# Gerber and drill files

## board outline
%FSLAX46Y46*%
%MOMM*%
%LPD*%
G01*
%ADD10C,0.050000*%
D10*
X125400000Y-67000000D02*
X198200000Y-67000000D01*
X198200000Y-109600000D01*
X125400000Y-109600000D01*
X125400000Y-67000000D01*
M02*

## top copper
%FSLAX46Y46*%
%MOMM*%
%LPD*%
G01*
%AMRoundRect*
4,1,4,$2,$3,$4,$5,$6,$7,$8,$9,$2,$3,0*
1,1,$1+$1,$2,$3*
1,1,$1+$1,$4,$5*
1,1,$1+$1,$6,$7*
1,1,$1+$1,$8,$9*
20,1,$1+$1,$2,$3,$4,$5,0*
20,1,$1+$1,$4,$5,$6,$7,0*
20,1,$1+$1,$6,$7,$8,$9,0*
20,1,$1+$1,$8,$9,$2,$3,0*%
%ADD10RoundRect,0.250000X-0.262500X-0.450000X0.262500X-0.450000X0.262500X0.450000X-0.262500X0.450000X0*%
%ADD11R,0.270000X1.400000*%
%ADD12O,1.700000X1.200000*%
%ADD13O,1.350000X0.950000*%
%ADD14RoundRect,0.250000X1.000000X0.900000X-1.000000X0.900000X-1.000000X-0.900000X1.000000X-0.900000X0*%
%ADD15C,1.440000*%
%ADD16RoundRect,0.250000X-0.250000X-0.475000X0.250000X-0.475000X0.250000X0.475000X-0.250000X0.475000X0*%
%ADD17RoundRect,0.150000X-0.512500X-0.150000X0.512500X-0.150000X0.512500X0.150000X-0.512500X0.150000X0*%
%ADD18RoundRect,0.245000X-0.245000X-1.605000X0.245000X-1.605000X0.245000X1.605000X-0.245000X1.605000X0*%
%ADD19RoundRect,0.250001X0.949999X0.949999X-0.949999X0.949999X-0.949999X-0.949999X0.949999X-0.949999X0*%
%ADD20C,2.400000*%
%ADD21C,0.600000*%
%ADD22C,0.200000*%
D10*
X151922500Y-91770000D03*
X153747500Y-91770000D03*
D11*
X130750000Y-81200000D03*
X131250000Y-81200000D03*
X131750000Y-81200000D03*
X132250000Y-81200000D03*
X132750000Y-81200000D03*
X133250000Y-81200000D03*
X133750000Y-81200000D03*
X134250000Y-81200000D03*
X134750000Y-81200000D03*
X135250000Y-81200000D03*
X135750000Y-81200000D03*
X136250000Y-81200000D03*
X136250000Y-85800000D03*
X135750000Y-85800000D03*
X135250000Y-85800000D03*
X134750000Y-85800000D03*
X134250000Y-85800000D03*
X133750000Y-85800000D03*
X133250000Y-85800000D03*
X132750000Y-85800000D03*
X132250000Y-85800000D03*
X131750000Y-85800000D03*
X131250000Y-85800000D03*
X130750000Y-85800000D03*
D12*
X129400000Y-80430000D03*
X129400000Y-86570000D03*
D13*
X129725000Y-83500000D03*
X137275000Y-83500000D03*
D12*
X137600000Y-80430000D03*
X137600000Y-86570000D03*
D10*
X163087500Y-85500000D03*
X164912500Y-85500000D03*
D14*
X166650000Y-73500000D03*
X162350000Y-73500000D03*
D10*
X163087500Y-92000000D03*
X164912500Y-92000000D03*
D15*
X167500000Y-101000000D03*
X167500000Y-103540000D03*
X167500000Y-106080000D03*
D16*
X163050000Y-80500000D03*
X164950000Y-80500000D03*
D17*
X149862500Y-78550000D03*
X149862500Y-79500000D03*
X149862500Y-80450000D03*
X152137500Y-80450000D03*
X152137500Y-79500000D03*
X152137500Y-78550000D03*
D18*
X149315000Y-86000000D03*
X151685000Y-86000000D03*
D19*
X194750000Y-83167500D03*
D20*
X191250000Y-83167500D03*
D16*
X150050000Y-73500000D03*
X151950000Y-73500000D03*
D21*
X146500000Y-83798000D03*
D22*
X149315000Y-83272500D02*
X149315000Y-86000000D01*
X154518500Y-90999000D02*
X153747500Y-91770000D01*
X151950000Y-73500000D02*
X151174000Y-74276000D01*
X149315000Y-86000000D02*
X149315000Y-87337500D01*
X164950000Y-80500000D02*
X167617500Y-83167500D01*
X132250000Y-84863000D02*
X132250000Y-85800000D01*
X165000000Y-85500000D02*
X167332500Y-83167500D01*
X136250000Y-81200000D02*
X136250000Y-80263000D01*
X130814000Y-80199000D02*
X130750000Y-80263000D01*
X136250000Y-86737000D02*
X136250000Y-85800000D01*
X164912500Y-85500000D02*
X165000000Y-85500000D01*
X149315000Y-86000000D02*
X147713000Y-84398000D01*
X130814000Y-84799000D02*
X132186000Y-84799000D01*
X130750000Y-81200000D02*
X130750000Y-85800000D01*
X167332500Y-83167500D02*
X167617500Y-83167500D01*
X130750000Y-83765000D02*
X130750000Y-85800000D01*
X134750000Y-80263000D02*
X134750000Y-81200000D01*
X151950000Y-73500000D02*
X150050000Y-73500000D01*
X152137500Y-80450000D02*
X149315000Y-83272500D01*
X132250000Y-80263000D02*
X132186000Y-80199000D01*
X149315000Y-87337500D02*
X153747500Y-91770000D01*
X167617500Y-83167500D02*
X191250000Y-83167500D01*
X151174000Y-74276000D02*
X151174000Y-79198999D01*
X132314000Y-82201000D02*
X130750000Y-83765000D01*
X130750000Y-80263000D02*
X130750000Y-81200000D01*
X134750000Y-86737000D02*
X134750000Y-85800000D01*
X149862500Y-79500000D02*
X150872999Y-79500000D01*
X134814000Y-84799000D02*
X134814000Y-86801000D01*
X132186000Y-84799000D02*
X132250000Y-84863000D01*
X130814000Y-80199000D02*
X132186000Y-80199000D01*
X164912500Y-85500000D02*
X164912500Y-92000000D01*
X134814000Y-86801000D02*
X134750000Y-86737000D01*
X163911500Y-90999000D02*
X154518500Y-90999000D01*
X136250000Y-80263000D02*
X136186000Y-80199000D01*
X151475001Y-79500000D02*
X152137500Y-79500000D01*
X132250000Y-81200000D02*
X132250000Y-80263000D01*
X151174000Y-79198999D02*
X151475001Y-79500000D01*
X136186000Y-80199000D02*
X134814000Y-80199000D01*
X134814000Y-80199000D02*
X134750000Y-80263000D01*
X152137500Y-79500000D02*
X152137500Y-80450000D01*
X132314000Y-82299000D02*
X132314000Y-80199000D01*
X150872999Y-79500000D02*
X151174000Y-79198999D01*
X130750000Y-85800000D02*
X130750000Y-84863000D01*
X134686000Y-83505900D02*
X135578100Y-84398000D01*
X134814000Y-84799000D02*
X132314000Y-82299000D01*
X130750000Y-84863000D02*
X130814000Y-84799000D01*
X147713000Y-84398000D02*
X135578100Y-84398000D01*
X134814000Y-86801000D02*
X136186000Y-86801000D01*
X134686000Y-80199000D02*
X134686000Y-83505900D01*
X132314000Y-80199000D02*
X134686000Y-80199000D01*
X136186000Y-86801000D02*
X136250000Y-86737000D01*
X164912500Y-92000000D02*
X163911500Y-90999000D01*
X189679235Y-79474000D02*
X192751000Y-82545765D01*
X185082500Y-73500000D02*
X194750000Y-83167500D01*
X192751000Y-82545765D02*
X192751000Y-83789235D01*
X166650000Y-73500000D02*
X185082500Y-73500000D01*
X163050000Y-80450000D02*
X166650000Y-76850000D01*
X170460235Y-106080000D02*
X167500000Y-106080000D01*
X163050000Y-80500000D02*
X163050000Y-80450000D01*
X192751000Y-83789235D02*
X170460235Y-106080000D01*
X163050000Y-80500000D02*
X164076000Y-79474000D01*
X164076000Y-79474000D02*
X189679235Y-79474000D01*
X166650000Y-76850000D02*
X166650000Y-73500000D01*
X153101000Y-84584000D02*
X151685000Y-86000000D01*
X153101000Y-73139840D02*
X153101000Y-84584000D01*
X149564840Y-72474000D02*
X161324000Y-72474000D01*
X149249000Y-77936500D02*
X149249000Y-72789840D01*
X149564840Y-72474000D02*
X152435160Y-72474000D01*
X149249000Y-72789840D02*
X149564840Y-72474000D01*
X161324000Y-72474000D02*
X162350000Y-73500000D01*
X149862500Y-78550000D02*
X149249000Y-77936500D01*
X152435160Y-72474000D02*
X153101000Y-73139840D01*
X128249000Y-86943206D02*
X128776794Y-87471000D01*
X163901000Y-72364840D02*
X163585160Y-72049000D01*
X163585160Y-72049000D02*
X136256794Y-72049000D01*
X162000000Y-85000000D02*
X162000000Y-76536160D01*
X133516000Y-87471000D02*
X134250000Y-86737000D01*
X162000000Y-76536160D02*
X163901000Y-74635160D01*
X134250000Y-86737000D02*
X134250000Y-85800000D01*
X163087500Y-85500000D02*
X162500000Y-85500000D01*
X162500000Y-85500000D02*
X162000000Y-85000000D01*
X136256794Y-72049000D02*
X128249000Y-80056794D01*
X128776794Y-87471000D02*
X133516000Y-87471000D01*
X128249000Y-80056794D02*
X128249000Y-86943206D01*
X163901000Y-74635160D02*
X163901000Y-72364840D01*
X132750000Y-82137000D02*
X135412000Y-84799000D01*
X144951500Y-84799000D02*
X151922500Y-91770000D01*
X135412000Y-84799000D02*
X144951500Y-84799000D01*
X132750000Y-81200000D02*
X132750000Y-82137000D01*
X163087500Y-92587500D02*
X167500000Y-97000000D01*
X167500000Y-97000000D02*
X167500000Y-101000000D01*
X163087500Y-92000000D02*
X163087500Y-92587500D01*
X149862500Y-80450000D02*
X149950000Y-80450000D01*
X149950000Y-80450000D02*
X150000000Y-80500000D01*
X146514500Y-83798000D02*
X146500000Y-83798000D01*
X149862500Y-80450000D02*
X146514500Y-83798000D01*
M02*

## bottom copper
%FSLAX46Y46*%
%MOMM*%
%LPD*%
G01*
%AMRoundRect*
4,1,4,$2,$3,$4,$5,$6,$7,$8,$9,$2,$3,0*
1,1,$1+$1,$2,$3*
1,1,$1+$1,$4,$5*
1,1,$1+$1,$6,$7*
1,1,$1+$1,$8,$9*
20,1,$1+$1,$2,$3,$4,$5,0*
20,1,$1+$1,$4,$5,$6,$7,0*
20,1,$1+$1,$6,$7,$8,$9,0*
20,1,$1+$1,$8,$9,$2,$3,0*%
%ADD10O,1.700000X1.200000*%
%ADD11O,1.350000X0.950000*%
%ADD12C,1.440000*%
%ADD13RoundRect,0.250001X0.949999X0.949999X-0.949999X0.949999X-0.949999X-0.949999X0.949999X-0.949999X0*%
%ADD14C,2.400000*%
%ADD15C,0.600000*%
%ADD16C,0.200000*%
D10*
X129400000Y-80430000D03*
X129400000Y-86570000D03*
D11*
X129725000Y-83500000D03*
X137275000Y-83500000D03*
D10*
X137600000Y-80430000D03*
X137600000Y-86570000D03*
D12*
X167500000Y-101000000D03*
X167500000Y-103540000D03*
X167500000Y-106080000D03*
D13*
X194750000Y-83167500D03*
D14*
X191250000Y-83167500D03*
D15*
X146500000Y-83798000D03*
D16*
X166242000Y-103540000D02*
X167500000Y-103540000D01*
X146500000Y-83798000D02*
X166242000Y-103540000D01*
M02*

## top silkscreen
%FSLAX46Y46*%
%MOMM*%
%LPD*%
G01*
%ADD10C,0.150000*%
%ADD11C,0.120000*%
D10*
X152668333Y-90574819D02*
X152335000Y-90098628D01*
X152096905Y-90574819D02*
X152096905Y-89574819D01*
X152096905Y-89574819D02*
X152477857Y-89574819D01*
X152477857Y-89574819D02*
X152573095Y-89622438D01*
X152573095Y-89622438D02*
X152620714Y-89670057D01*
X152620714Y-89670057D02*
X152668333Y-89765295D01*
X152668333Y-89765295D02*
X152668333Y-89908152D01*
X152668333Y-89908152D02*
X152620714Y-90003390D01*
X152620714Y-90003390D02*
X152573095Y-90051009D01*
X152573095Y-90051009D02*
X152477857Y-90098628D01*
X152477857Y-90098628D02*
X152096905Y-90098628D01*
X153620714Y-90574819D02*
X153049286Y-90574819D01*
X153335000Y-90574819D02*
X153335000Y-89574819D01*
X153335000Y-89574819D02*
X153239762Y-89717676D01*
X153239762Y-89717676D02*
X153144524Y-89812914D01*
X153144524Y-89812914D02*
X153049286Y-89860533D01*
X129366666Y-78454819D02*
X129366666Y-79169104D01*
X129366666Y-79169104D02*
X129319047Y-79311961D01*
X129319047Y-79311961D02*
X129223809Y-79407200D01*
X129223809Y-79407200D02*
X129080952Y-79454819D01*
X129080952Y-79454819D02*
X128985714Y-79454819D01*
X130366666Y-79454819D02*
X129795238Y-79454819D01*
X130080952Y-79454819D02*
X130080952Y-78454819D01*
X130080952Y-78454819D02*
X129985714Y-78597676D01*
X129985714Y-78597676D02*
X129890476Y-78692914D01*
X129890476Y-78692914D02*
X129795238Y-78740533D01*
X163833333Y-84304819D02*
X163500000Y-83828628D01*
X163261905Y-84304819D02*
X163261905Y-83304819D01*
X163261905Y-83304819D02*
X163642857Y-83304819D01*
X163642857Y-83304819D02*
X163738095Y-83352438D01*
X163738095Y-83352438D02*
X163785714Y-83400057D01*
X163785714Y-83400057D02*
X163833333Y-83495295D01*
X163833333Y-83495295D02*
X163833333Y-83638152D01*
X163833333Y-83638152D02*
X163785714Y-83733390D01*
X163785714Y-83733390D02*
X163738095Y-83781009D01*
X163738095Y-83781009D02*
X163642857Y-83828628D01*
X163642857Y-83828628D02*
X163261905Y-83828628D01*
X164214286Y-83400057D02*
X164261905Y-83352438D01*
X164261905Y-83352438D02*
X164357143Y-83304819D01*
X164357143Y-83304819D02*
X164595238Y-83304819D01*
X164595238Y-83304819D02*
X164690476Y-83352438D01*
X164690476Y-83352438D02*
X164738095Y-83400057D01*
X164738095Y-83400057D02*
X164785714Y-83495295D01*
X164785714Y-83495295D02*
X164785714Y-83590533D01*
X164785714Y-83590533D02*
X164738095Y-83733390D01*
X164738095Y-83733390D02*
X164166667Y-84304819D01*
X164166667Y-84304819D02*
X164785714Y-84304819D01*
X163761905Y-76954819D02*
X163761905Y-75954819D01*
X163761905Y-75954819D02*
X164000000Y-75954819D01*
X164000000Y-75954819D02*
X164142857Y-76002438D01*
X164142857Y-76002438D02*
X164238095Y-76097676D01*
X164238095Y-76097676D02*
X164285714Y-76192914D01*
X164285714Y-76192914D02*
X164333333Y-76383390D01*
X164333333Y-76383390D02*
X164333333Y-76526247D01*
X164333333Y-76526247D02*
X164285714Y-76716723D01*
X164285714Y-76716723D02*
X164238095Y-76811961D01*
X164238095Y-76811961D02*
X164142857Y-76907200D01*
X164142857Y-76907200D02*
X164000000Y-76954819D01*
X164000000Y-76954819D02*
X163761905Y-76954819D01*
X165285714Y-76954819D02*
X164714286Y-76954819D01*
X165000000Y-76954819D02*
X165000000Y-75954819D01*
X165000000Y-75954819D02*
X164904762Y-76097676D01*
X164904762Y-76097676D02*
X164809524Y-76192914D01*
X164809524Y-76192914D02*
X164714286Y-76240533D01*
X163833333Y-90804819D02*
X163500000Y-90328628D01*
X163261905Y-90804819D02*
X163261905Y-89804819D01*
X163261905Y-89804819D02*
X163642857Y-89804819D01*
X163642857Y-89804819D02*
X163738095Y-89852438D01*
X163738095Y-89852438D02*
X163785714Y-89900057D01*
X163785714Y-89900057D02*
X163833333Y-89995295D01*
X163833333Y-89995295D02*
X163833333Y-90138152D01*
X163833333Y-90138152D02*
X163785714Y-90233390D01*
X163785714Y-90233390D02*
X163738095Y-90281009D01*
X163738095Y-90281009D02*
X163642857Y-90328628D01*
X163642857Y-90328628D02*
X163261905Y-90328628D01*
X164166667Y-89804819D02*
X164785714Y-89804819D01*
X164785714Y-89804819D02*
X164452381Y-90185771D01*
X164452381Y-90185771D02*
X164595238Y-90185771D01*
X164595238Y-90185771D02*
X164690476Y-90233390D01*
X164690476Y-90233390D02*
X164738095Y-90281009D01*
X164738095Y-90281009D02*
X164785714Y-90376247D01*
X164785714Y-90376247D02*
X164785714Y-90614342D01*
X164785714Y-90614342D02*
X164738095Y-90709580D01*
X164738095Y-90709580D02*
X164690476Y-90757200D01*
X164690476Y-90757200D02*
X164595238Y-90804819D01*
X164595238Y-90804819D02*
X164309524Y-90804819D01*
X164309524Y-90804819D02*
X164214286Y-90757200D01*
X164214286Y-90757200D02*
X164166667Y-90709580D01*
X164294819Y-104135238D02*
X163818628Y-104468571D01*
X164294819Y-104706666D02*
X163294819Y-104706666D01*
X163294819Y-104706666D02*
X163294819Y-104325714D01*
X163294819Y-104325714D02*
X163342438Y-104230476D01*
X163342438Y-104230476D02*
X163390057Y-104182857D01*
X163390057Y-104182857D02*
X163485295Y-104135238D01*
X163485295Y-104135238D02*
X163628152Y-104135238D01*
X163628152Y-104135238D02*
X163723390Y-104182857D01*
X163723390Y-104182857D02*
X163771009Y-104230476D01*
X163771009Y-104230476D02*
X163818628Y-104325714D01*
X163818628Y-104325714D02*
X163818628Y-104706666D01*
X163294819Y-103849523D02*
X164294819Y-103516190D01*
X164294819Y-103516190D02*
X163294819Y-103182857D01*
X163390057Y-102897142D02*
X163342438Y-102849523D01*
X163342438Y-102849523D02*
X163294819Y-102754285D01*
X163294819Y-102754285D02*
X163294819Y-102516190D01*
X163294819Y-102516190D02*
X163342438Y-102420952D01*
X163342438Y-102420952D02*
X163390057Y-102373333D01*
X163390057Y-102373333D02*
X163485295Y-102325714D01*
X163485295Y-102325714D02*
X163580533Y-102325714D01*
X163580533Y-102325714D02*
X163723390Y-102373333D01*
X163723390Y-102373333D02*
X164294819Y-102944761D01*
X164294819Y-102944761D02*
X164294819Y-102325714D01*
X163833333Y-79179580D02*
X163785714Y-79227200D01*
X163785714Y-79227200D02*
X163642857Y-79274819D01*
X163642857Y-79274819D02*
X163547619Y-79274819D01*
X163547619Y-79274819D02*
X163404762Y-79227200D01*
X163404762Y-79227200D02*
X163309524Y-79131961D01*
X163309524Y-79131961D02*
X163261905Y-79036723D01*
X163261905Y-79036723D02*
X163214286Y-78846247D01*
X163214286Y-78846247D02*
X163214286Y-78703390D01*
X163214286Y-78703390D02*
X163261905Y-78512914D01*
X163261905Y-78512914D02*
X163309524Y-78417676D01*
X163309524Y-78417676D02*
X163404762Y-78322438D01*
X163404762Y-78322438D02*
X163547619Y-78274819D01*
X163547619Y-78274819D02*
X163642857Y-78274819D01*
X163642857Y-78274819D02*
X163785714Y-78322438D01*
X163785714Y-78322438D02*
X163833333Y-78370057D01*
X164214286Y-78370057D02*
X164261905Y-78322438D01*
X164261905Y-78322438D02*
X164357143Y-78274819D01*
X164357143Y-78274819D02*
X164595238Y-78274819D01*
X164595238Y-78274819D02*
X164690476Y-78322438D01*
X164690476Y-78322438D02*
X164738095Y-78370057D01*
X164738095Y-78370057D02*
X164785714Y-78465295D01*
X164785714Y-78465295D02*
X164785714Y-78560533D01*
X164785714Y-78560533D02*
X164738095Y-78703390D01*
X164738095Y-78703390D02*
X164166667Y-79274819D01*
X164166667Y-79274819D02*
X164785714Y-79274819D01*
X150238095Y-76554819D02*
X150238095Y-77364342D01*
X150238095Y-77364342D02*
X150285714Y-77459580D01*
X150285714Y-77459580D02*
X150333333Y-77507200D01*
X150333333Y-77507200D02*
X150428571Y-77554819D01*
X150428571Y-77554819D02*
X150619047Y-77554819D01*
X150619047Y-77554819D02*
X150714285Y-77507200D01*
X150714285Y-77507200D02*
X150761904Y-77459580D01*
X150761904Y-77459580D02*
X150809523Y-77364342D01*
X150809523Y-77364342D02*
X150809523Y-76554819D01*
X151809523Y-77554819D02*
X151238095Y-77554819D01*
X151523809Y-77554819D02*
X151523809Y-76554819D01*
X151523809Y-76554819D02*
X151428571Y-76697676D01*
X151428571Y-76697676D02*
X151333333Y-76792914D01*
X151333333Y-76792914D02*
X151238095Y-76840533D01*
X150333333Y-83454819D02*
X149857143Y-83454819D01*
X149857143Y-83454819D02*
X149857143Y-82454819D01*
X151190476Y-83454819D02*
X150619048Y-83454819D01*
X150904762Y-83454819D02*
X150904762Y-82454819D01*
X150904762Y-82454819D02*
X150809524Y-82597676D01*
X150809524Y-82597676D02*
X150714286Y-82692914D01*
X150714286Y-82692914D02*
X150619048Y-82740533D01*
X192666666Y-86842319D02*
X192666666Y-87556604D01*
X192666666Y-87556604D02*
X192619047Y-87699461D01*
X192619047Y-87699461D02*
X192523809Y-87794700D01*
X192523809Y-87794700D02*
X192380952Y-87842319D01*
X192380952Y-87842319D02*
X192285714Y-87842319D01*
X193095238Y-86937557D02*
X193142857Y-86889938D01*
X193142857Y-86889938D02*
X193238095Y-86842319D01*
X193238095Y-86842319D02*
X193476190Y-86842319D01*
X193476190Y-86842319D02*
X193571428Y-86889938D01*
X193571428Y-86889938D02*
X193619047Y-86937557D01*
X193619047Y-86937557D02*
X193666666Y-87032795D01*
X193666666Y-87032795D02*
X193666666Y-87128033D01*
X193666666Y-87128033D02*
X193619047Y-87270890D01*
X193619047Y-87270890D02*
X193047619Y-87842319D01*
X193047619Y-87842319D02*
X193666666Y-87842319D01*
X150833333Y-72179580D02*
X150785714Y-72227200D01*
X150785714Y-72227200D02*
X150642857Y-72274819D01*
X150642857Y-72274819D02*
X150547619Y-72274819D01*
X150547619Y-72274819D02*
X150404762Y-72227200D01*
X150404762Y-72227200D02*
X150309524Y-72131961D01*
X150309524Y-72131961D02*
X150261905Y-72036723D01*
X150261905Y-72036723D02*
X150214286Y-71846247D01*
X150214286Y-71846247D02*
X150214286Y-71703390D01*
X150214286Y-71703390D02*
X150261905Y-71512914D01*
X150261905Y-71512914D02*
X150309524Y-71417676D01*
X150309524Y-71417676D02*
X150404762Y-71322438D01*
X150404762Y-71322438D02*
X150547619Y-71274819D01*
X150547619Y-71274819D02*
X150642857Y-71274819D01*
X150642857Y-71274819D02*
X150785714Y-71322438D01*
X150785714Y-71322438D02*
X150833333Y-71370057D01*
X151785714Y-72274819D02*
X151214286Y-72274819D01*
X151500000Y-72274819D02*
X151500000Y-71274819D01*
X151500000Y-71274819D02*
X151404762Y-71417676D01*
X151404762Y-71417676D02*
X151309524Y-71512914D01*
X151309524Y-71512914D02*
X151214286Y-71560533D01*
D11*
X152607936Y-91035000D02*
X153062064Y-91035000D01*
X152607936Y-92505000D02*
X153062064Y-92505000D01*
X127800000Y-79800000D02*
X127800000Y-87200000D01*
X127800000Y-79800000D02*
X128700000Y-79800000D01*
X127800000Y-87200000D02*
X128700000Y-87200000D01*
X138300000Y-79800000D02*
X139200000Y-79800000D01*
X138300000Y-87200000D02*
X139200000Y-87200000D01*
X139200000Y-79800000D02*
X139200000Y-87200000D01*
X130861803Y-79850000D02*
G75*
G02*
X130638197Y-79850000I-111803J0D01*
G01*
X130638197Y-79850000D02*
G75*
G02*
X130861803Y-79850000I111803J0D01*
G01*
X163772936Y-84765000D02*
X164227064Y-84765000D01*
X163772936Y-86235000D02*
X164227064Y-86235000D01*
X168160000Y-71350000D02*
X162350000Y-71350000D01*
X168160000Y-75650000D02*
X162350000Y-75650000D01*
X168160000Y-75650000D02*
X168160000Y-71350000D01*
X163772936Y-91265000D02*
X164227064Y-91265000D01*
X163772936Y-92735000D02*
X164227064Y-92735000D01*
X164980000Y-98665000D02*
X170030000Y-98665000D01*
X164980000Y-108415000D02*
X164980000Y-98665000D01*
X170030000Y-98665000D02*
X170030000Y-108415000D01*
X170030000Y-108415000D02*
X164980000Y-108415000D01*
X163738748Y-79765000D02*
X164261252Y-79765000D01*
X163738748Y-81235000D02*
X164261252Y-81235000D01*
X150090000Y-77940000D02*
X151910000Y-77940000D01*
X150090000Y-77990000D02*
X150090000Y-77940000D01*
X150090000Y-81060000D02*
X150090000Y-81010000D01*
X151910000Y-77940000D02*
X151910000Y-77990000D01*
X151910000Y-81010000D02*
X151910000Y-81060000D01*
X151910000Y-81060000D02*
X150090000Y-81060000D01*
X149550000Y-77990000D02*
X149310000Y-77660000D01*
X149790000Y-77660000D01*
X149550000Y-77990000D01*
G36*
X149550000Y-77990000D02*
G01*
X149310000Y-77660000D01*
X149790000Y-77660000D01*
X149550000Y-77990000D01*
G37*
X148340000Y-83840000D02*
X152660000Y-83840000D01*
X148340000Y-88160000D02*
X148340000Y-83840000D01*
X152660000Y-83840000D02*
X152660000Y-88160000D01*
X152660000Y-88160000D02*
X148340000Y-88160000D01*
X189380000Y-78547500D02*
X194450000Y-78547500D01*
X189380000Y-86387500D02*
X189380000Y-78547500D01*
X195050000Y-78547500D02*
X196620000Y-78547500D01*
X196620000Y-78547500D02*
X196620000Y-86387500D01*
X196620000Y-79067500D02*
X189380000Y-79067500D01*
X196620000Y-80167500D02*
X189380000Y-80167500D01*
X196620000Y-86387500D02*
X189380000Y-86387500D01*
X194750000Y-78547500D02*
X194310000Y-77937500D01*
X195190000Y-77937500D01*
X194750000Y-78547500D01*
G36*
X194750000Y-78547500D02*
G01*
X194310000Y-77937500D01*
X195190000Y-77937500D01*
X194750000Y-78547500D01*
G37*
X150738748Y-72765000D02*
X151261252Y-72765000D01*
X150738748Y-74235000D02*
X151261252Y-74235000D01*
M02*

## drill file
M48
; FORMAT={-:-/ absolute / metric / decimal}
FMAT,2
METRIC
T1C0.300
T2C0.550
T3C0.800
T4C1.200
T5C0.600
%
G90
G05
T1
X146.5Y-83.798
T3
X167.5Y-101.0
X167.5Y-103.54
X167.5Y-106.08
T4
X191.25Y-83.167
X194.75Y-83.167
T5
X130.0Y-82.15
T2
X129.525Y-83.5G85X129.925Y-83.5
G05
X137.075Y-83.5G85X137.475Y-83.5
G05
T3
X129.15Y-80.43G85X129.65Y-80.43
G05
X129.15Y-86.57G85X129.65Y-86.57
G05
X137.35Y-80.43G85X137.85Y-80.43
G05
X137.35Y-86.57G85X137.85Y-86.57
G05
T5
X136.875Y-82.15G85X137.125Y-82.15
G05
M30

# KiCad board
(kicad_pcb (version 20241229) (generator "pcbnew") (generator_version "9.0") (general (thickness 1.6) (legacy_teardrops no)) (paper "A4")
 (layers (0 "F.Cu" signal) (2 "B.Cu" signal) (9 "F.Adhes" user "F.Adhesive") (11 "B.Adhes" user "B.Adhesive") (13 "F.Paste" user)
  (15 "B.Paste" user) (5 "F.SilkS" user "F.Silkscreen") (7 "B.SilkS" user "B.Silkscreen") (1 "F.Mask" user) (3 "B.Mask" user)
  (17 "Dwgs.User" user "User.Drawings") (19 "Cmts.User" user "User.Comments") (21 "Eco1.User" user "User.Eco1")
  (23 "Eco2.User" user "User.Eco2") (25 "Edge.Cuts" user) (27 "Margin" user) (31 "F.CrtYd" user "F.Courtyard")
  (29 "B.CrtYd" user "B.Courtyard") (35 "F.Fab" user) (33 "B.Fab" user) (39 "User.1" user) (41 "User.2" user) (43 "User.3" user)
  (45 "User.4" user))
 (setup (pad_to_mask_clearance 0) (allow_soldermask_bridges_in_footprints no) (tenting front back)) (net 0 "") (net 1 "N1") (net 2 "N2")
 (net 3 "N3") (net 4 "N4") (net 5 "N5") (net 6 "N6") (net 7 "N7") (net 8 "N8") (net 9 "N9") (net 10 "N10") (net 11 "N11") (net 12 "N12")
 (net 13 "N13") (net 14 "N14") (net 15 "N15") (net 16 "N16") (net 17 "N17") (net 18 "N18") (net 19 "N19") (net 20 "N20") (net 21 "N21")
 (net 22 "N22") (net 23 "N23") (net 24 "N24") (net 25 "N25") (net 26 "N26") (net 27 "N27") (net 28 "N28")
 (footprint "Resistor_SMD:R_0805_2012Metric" (layer "F.Cu") (at 152.835 91.77)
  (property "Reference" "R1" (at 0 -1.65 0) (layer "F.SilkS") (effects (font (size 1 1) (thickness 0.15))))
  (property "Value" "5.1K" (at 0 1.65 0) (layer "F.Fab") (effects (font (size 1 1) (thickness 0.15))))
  (fp_line (start -0.227064 -0.735) (end 0.227064 -0.735) (stroke (width 0.12) (type solid)) (layer "F.SilkS"))
  (fp_line (start -0.227064 0.735) (end 0.227064 0.735) (stroke (width 0.12) (type solid)) (layer "F.SilkS"))
  (pad "1" smd roundrect (at -0.9125 0) (size 1.025 1.4) (layers "F.Cu" "F.Mask" "F.Paste") (roundrect_rratio 0.243902) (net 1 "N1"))
  (pad "2" smd roundrect (at 0.9125 0) (size 1.025 1.4) (layers "F.Cu" "F.Mask" "F.Paste") (roundrect_rratio 0.243902) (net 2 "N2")))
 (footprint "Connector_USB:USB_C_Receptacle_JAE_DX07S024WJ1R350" (layer "F.Cu") (at 133.5 83.5)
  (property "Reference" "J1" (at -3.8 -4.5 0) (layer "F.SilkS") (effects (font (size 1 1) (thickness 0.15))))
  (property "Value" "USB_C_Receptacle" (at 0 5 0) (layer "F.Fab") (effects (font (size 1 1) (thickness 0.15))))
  (fp_line (start -5.7 -3.7) (end -5.7 3.7) (stroke (width 0.12) (type solid)) (layer "F.SilkS"))
  (fp_line (start -5.7 -3.7) (end -4.8 -3.7) (stroke (width 0.12) (type solid)) (layer "F.SilkS"))
  (fp_line (start -5.7 3.7) (end -4.8 3.7) (stroke (width 0.12) (type solid)) (layer "F.SilkS"))
  (fp_line (start 4.8 -3.7) (end 5.7 -3.7) (stroke (width 0.12) (type solid)) (layer "F.SilkS"))
  (fp_line (start 4.8 3.7) (end 5.7 3.7) (stroke (width 0.12) (type solid)) (layer "F.SilkS"))
  (fp_line (start 5.7 -3.7) (end 5.7 3.7) (stroke (width 0.12) (type solid)) (layer "F.SilkS"))
  (fp_circle (center -2.75 -3.65) (end -2.638197 -3.65) (stroke (width 0.12) (type solid)) (fill no) (layer "F.SilkS"))
  (pad "" np_thru_hole circle (at -3.5 -1.35) (size 0.6 0.6) (drill 0.6) (layers "*.Cu" "*.Mask"))
  (pad "" np_thru_hole oval (at 3.5 -1.35) (size 0.85 0.6) (drill oval 0.85 0.6) (layers "*.Cu" "*.Mask"))
  (pad "A1" smd rect (at -2.75 -2.3) (size 0.27 1.4) (layers "F.Cu" "F.Mask" "F.Paste") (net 2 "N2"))
  (pad "A2" smd rect (at -2.25 -2.3) (size 0.27 1.4) (layers "F.Cu" "F.Mask" "F.Paste") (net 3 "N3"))
  (pad "A3" smd rect (at -1.75 -2.3) (size 0.27 1.4) (layers "F.Cu" "F.Mask" "F.Paste") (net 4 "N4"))
  (pad "A4" smd rect (at -1.25 -2.3) (size 0.27 1.4) (layers "F.Cu" "F.Mask" "F.Paste") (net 2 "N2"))
  (pad "A5" smd rect (at -0.75 -2.3) (size 0.27 1.4) (layers "F.Cu" "F.Mask" "F.Paste") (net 1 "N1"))
  (pad "A6" smd rect (at -0.25 -2.3) (size 0.27 1.4) (layers "F.Cu" "F.Mask" "F.Paste") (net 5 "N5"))
  (pad "A7" smd rect (at 0.25 -2.3) (size 0.27 1.4) (layers "F.Cu" "F.Mask" "F.Paste") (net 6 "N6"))
  (pad "A8" smd rect (at 0.75 -2.3) (size 0.27 1.4) (layers "F.Cu" "F.Mask" "F.Paste") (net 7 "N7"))
  (pad "A9" smd rect (at 1.25 -2.3) (size 0.27 1.4) (layers "F.Cu" "F.Mask" "F.Paste") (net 2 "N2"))
  (pad "A10" smd rect (at 1.75 -2.3) (size 0.27 1.4) (layers "F.Cu" "F.Mask" "F.Paste") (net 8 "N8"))
  (pad "A11" smd rect (at 2.25 -2.3) (size 0.27 1.4) (layers "F.Cu" "F.Mask" "F.Paste") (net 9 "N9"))
  (pad "A12" smd rect (at 2.75 -2.3) (size 0.27 1.4) (layers "F.Cu" "F.Mask" "F.Paste") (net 2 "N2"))
  (pad "B1" smd rect (at 2.75 2.3) (size 0.27 1.4) (layers "F.Cu" "F.Mask" "F.Paste") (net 2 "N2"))
  (pad "B2" smd rect (at 2.25 2.3) (size 0.27 1.4) (layers "F.Cu" "F.Mask" "F.Paste") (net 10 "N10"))
  (pad "B3" smd rect (at 1.75 2.3) (size 0.27 1.4) (layers "F.Cu" "F.Mask" "F.Paste") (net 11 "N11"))
  (pad "B4" smd rect (at 1.25 2.3) (size 0.27 1.4) (layers "F.Cu" "F.Mask" "F.Paste") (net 2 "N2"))
  (pad "B5" smd rect (at 0.75 2.3) (size 0.27 1.4) (layers "F.Cu" "F.Mask" "F.Paste") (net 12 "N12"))
  (pad "B6" smd rect (at 0.25 2.3) (size 0.27 1.4) (layers "F.Cu" "F.Mask" "F.Paste") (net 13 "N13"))
  (pad "B7" smd rect (at -0.25 2.3) (size 0.27 1.4) (layers "F.Cu" "F.Mask" "F.Paste") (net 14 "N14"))
  (pad "B8" smd rect (at -0.75 2.3) (size 0.27 1.4) (layers "F.Cu" "F.Mask" "F.Paste") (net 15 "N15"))
  (pad "B9" smd rect (at -1.25 2.3) (size 0.27 1.4) (layers "F.Cu" "F.Mask" "F.Paste") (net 2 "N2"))
  (pad "B10" smd rect (at -1.75 2.3) (size 0.27 1.4) (layers "F.Cu" "F.Mask" "F.Paste") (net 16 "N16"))
  (pad "B11" smd rect (at -2.25 2.3) (size 0.27 1.4) (layers "F.Cu" "F.Mask" "F.Paste") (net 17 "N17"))
  (pad "B12" smd rect (at -2.75 2.3) (size 0.27 1.4) (layers "F.Cu" "F.Mask" "F.Paste") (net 2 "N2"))
  (pad "S1" thru_hole oval (at -4.1 -3.07 90) (size 1.2 1.7) (drill oval 0.8 1.3) (layers "*.Cu" "*.Mask") (remove_unused_layers no)
   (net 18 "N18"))
  (pad "S1" thru_hole oval (at -4.1 3.07 90) (size 1.2 1.7) (drill oval 0.8 1.3) (layers "*.Cu" "*.Mask") (remove_unused_layers no)
   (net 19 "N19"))
  (pad "S1" thru_hole oval (at -3.775 0 90) (size 0.95 1.35) (drill oval 0.55 0.95) (layers "*.Cu" "*.Mask") (remove_unused_layers no)
   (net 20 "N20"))
  (pad "S1" thru_hole oval (at 3.775 0 90) (size 0.95 1.35) (drill oval 0.55 0.95) (layers "*.Cu" "*.Mask") (remove_unused_layers no)
   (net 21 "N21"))
  (pad "S1" thru_hole oval (at 4.1 -3.07 90) (size 1.2 1.7) (drill oval 0.8 1.3) (layers "*.Cu" "*.Mask") (remove_unused_layers no)
   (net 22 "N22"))
  (pad "S1" thru_hole oval (at 4.1 3.07 90) (size 1.2 1.7) (drill oval 0.8 1.3) (layers "*.Cu" "*.Mask") (remove_unused_layers no)
   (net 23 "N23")))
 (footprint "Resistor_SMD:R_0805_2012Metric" (layer "F.Cu") (at 164 85.5)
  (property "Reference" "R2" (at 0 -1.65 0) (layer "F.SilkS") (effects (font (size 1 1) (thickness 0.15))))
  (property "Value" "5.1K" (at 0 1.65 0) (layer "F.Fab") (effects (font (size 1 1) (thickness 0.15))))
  (fp_line (start -0.227064 -0.735) (end 0.227064 -0.735) (stroke (width 0.12) (type solid)) (layer "F.SilkS"))
  (fp_line (start -0.227064 0.735) (end 0.227064 0.735) (stroke (width 0.12) (type solid)) (layer "F.SilkS"))
  (pad "1" smd roundrect (at -0.9125 0) (size 1.025 1.4) (layers "F.Cu" "F.Mask" "F.Paste") (roundrect_rratio 0.243902) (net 12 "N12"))
  (pad "2" smd roundrect (at 0.9125 0) (size 1.025 1.4) (layers "F.Cu" "F.Mask" "F.Paste") (roundrect_rratio 0.243902) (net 2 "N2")))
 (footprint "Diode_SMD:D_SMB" (layer "F.Cu") (at 164.5 73.5 180)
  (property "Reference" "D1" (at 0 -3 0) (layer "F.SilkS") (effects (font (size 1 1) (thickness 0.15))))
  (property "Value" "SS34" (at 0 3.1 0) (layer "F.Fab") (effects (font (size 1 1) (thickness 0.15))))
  (fp_line (start -3.66 2.15) (end 2.15 2.15) (stroke (width 0.12) (type solid)) (layer "F.SilkS"))
  (fp_line (start -3.66 -2.15) (end 2.15 -2.15) (stroke (width 0.12) (type solid)) (layer "F.SilkS"))
  (fp_line (start -3.66 -2.15) (end -3.66 2.15) (stroke (width 0.12) (type solid)) (layer "F.SilkS"))
  (pad "1" smd roundrect (at -2.15 0 180) (size 2.5 2.3) (layers "F.Cu" "F.Mask" "F.Paste") (roundrect_rratio 0.1086956522) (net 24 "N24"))
  (pad "2" smd roundrect (at 2.15 0 180) (size 2.5 2.3) (layers "F.Cu" "F.Mask" "F.Paste") (roundrect_rratio 0.1086956522) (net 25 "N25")))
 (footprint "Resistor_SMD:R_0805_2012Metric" (layer "F.Cu") (at 164 92)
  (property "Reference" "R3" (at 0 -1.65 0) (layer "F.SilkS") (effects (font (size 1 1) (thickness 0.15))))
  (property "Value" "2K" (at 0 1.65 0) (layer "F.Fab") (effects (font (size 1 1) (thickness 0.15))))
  (fp_line (start -0.227064 -0.735) (end 0.227064 -0.735) (stroke (width 0.12) (type solid)) (layer "F.SilkS"))
  (fp_line (start -0.227064 0.735) (end 0.227064 0.735) (stroke (width 0.12) (type solid)) (layer "F.SilkS"))
  (pad "1" smd roundrect (at -0.9125 0) (size 1.025 1.4) (layers "F.Cu" "F.Mask" "F.Paste") (roundrect_rratio 0.243902) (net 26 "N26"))
  (pad "2" smd roundrect (at 0.9125 0) (size 1.025 1.4) (layers "F.Cu" "F.Mask" "F.Paste") (roundrect_rratio 0.243902) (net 2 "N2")))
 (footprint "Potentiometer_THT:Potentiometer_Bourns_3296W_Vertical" (layer "F.Cu") (at 167.5 101 90)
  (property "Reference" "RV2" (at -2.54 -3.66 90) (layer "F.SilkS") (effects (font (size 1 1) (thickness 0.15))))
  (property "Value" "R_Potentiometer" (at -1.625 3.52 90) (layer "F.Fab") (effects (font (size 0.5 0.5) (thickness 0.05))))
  (fp_line (start 2.335 -2.52) (end 2.335 2.53) (stroke (width 0.12) (type solid)) (layer "F.SilkS"))
  (fp_line (start -7.415 -2.52) (end 2.335 -2.52) (stroke (width 0.12) (type solid)) (layer "F.SilkS"))
  (fp_line (start 2.335 2.53) (end -7.415 2.53) (stroke (width 0.12) (type solid)) (layer "F.SilkS"))
  (fp_line (start -7.415 2.53) (end -7.415 -2.52) (stroke (width 0.12) (type solid)) (layer "F.SilkS"))
  (pad "1" thru_hole circle (at 0 0 90) (size 1.44 1.44) (drill 0.8) (layers "*.Cu" "*.Mask") (remove_unused_layers no) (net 26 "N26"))
  (pad "2" thru_hole circle (at -2.54 0 90) (size 1.44 1.44) (drill 0.8) (layers "*.Cu" "*.Mask") (remove_unused_layers no) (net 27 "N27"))
  (pad "3" thru_hole circle (at -5.08 0 90) (size 1.44 1.44) (drill 0.8) (layers "*.Cu" "*.Mask") (remove_unused_layers no) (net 24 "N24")))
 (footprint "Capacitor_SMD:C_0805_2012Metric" (layer "F.Cu") (at 164 80.5)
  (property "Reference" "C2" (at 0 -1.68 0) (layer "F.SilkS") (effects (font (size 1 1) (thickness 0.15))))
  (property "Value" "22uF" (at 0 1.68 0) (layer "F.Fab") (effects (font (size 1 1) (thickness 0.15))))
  (fp_line (start -0.261252 -0.735) (end 0.261252 -0.735) (stroke (width 0.12) (type solid)) (layer "F.SilkS"))
  (fp_line (start -0.261252 0.735) (end 0.261252 0.735) (stroke (width 0.12) (type solid)) (layer "F.SilkS"))
  (pad "1" smd roundrect (at -0.95 0) (size 1 1.45) (layers "F.Cu" "F.Mask" "F.Paste") (roundrect_rratio 0.25) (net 24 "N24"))
  (pad "2" smd roundrect (at 0.95 0) (size 1 1.45) (layers "F.Cu" "F.Mask" "F.Paste") (roundrect_rratio 0.25) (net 2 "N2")))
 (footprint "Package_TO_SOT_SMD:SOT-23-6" (layer "F.Cu") (at 151 79.5)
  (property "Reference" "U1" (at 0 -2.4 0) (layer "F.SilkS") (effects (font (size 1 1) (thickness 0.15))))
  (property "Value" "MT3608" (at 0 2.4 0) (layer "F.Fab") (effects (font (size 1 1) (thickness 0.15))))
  (fp_line (start -0.91 -1.56) (end 0.91 -1.56) (stroke (width 0.12) (type solid)) (layer "F.SilkS"))
  (fp_line (start -0.91 -1.51) (end -0.91 -1.56) (stroke (width 0.12) (type solid)) (layer "F.SilkS"))
  (fp_line (start -0.91 1.56) (end -0.91 1.51) (stroke (width 0.12) (type solid)) (layer "F.SilkS"))
  (fp_line (start 0.91 -1.56) (end 0.91 -1.51) (stroke (width 0.12) (type solid)) (layer "F.SilkS"))
  (fp_line (start 0.91 1.51) (end 0.91 1.56) (stroke (width 0.12) (type solid)) (layer "F.SilkS"))
  (fp_line (start 0.91 1.56) (end -0.91 1.56) (stroke (width 0.12) (type solid)) (layer "F.SilkS"))
  (fp_poly (pts (xy -1.45 -1.51) (xy -1.69 -1.84) (xy -1.21 -1.84)) (stroke (width 0.12) (type solid)) (fill yes) (layer "F.SilkS"))
  (pad "1" smd roundrect (at -1.1375 -0.95) (size 1.325 0.6) (layers "F.Cu" "F.Mask" "F.Paste") (roundrect_rratio 0.25) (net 25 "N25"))
  (pad "2" smd roundrect (at -1.1375 0) (size 1.325 0.6) (layers "F.Cu" "F.Mask" "F.Paste") (roundrect_rratio 0.25) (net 2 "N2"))
  (pad "3" smd roundrect (at -1.1375 0.95) (size 1.325 0.6) (layers "F.Cu" "F.Mask" "F.Paste") (roundrect_rratio 0.25) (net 27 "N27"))
  (pad "4" smd roundrect (at 1.1375 0.95) (size 1.325 0.6) (layers "F.Cu" "F.Mask" "F.Paste") (roundrect_rratio 0.25) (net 2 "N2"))
  (pad "5" smd roundrect (at 1.1375 0) (size 1.325 0.6) (layers "F.Cu" "F.Mask" "F.Paste") (roundrect_rratio 0.25) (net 2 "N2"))
  (pad "6" smd roundrect (at 1.1375 -0.95) (size 1.325 0.6) (layers "F.Cu" "F.Mask" "F.Paste") (roundrect_rratio 0.25) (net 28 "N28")))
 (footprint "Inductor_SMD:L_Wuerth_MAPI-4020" (layer "F.Cu") (at 150.5 86)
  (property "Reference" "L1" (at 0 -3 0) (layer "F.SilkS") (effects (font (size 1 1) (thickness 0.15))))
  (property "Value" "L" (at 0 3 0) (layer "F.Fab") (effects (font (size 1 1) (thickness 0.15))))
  (fp_line (start -2.16 -2.16) (end 2.16 -2.16) (stroke (width 0.12) (type solid)) (layer "F.SilkS"))
  (fp_line (start -2.16 2.16) (end -2.16 -2.16) (stroke (width 0.12) (type solid)) (layer "F.SilkS"))
  (fp_line (start 2.16 -2.16) (end 2.16 2.16) (stroke (width 0.12) (type solid)) (layer "F.SilkS"))
  (fp_line (start 2.16 2.16) (end -2.16 2.16) (stroke (width 0.12) (type solid)) (layer "F.SilkS"))
  (pad "1" smd roundrect (at -1.185 0) (size 0.98 3.7) (layers "F.Cu" "F.Mask" "F.Paste") (roundrect_rratio 0.25) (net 2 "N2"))
  (pad "2" smd roundrect (at 1.185 0) (size 0.98 3.7) (layers "F.Cu" "F.Mask" "F.Paste") (roundrect_rratio 0.25) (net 25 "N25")))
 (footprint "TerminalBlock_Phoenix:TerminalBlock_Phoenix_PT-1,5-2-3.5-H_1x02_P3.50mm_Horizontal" (layer "F.Cu") (at 194.75 83.1675 180)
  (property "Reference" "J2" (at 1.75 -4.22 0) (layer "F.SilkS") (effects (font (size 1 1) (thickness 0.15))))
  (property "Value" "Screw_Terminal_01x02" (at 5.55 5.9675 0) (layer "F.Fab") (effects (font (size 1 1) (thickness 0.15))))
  (fp_line (start 5.37 4.62) (end 0.3 4.62) (stroke (width 0.12) (type solid)) (layer "F.SilkS"))
  (fp_line (start 5.37 -3.22) (end 5.37 4.62) (stroke (width 0.12) (type solid)) (layer "F.SilkS"))
  (fp_line (start -0.3 4.62) (end -1.87 4.62) (stroke (width 0.12) (type solid)) (layer "F.SilkS"))
  (fp_line (start -1.87 4.62) (end -1.87 -3.22) (stroke (width 0.12) (type solid)) (layer "F.SilkS"))
  (fp_line (start -1.87 4.1) (end 5.37 4.1) (stroke (width 0.12) (type solid)) (layer "F.SilkS"))
  (fp_line (start -1.87 3) (end 5.37 3) (stroke (width 0.12) (type solid)) (layer "F.SilkS"))
  (fp_line (start -1.87 -3.22) (end 5.37 -3.22) (stroke (width 0.12) (type solid)) (layer "F.SilkS"))
  (fp_poly (pts (xy 0 4.62) (xy 0.44 5.23) (xy -0.44 5.23)) (stroke (width 0.12) (type solid)) (fill yes) (layer "F.SilkS"))
  (pad "1" thru_hole roundrect (at 0 0 180) (size 2.4 2.4) (drill 1.2) (layers "*.Cu" "*.Mask") (remove_unused_layers no)
   (roundrect_rratio 0.104167) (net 24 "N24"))
  (pad "2" thru_hole circle (at 3.5 0 180) (size 2.4 2.4) (drill 1.2) (layers "*.Cu" "*.Mask") (remove_unused_layers no) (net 2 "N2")))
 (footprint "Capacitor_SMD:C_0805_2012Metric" (layer "F.Cu") (at 151 73.5)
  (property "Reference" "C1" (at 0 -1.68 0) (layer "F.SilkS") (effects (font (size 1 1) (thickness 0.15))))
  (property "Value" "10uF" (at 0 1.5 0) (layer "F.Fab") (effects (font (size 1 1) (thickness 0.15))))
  (fp_line (start -0.261252 -0.735) (end 0.261252 -0.735) (stroke (width 0.12) (type solid)) (layer "F.SilkS"))
  (fp_line (start -0.261252 0.735) (end 0.261252 0.735) (stroke (width 0.12) (type solid)) (layer "F.SilkS"))
  (pad "1" smd roundrect (at -0.95 0) (size 1 1.45) (layers "F.Cu" "F.Mask" "F.Paste") (roundrect_rratio 0.25) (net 2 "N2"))
  (pad "2" smd roundrect (at 0.95 0) (size 1 1.45) (layers "F.Cu" "F.Mask" "F.Paste") (roundrect_rratio 0.25) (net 2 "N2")))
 (gr_rect (start 125.4 67) (end 198.2 109.6) (stroke (width 0.05) (type default)) (fill no) (layer "Edge.Cuts"))
 (segment (start 149.315 83.2725) (end 149.315 86) (width 0.2) (layer "F.Cu") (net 2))
 (segment (start 154.5185 90.999) (end 153.7475 91.77) (width 0.2) (layer "F.Cu") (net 2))
 (segment (start 151.95 73.5) (end 151.174 74.276) (width 0.2) (layer "F.Cu") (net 2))
 (segment (start 149.315 86) (end 149.315 87.3375) (width 0.2) (layer "F.Cu") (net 2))
 (segment (start 164.95 80.5) (end 167.6175 83.1675) (width 0.2) (layer "F.Cu") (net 2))
 (segment (start 132.25 84.863) (end 132.25 85.8) (width 0.2) (layer "F.Cu") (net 2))
 (segment (start 165 85.5) (end 167.3325 83.1675) (width 0.2) (layer "F.Cu") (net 2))
 (segment (start 136.25 81.2) (end 136.25 80.263) (width 0.2) (layer "F.Cu") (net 2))
 (segment (start 130.814 80.199) (end 130.75 80.263) (width 0.2) (layer "F.Cu") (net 2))
 (segment (start 136.25 86.737) (end 136.25 85.8) (width 0.2) (layer "F.Cu") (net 2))
 (segment (start 164.9125 85.5) (end 165 85.5) (width 0.2) (layer "F.Cu") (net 2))
 (segment (start 149.315 86) (end 147.713 84.398) (width 0.2) (layer "F.Cu") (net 2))
 (segment (start 130.814 84.799) (end 132.186 84.799) (width 0.2) (layer "F.Cu") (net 2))
 (segment (start 130.75 81.2) (end 130.75 85.8) (width 0.2) (layer "F.Cu") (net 2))
 (segment (start 167.3325 83.1675) (end 167.6175 83.1675) (width 0.2) (layer "F.Cu") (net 2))
 (segment (start 130.75 83.765) (end 130.75 85.8) (width 0.2) (layer "F.Cu") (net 2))
 (segment (start 134.75 80.263) (end 134.75 81.2) (width 0.2) (layer "F.Cu") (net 2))
 (segment (start 151.95 73.5) (end 150.05 73.5) (width 0.2) (layer "F.Cu") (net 2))
 (segment (start 152.1375 80.45) (end 149.315 83.2725) (width 0.2) (layer "F.Cu") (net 2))
 (segment (start 132.25 80.263) (end 132.186 80.199) (width 0.2) (layer "F.Cu") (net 2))
 (segment (start 149.315 87.3375) (end 153.7475 91.77) (width 0.2) (layer "F.Cu") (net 2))
 (segment (start 167.6175 83.1675) (end 191.25 83.1675) (width 0.2) (layer "F.Cu") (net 2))
 (segment (start 151.174 74.276) (end 151.174 79.198999) (width 0.2) (layer "F.Cu") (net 2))
 (segment (start 132.314 82.201) (end 130.75 83.765) (width 0.2) (layer "F.Cu") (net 2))
 (segment (start 130.75 80.263) (end 130.75 81.2) (width 0.2) (layer "F.Cu") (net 2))
 (segment (start 134.75 86.737) (end 134.75 85.8) (width 0.2) (layer "F.Cu") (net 2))
 (segment (start 149.8625 79.5) (end 150.872999 79.5) (width 0.2) (layer "F.Cu") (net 2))
 (segment (start 134.814 84.799) (end 134.814 86.801) (width 0.2) (layer "F.Cu") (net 2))
 (segment (start 132.186 84.799) (end 132.25 84.863) (width 0.2) (layer "F.Cu") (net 2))
 (segment (start 130.814 80.199) (end 132.186 80.199) (width 0.2) (layer "F.Cu") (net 2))
 (segment (start 164.9125 85.5) (end 164.9125 92) (width 0.2) (layer "F.Cu") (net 2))
 (segment (start 134.814 86.801) (end 134.75 86.737) (width 0.2) (layer "F.Cu") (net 2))
 (segment (start 163.9115 90.999) (end 154.5185 90.999) (width 0.2) (layer "F.Cu") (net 2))
 (segment (start 136.25 80.263) (end 136.186 80.199) (width 0.2) (layer "F.Cu") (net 2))
 (segment (start 151.475001 79.5) (end 152.1375 79.5) (width 0.2) (layer "F.Cu") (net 2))
 (segment (start 132.25 81.2) (end 132.25 80.263) (width 0.2) (layer "F.Cu") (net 2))
 (segment (start 151.174 79.198999) (end 151.475001 79.5) (width 0.2) (layer "F.Cu") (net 2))
 (segment (start 136.186 80.199) (end 134.814 80.199) (width 0.2) (layer "F.Cu") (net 2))
 (segment (start 134.814 80.199) (end 134.75 80.263) (width 0.2) (layer "F.Cu") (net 2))
 (segment (start 152.1375 79.5) (end 152.1375 80.45) (width 0.2) (layer "F.Cu") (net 2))
 (segment (start 132.314 82.299) (end 132.314 80.199) (width 0.2) (layer "F.Cu") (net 2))
 (segment (start 150.872999 79.5) (end 151.174 79.198999) (width 0.2) (layer "F.Cu") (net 2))
 (segment (start 130.75 85.8) (end 130.75 84.863) (width 0.2) (layer "F.Cu") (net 2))
 (segment (start 134.686 83.5059) (end 135.5781 84.398) (width 0.2) (layer "F.Cu") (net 2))
 (segment (start 134.814 84.799) (end 132.314 82.299) (width 0.2) (layer "F.Cu") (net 2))
 (segment (start 130.75 84.863) (end 130.814 84.799) (width 0.2) (layer "F.Cu") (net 2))
 (segment (start 147.713 84.398) (end 135.5781 84.398) (width 0.2) (layer "F.Cu") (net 2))
 (segment (start 134.814 86.801) (end 136.186 86.801) (width 0.2) (layer "F.Cu") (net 2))
 (segment (start 134.686 80.199) (end 134.686 83.5059) (width 0.2) (layer "F.Cu") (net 2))
 (segment (start 132.314 80.199) (end 134.686 80.199) (width 0.2) (layer "F.Cu") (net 2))
 (segment (start 136.186 86.801) (end 136.25 86.737) (width 0.2) (layer "F.Cu") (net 2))
 (segment (start 164.9125 92) (end 163.9115 90.999) (width 0.2) (layer "F.Cu") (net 2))
 (segment (start 189.679235 79.474) (end 192.751 82.545765) (width 0.2) (layer "F.Cu") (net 24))
 (segment (start 185.0825 73.5) (end 194.75 83.1675) (width 0.2) (layer "F.Cu") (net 24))
 (segment (start 192.751 82.545765) (end 192.751 83.789235) (width 0.2) (layer "F.Cu") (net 24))
 (segment (start 166.65 73.5) (end 185.0825 73.5) (width 0.2) (layer "F.Cu") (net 24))
 (segment (start 163.05 80.45) (end 166.65 76.85) (width 0.2) (layer "F.Cu") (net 24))
 (segment (start 170.460235 106.08) (end 167.5 106.08) (width 0.2) (layer "F.Cu") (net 24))
 (segment (start 163.05 80.5) (end 163.05 80.45) (width 0.2) (layer "F.Cu") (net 24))
 (segment (start 192.751 83.789235) (end 170.460235 106.08) (width 0.2) (layer "F.Cu") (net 24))
 (segment (start 163.05 80.5) (end 164.076 79.474) (width 0.2) (layer "F.Cu") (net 24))
 (segment (start 164.076 79.474) (end 189.679235 79.474) (width 0.2) (layer "F.Cu") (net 24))
 (segment (start 166.65 76.85) (end 166.65 73.5) (width 0.2) (layer "F.Cu") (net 24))
 (segment (start 153.101 84.584) (end 151.685 86) (width 0.2) (layer "F.Cu") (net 25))
 (segment (start 153.101 73.13984) (end 153.101 84.584) (width 0.2) (layer "F.Cu") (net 25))
 (segment (start 149.56484 72.474) (end 161.324 72.474) (width 0.2) (layer "F.Cu") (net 25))
 (segment (start 149.249 77.9365) (end 149.249 72.78984) (width 0.2) (layer "F.Cu") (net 25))
 (segment (start 149.56484 72.474) (end 152.43516 72.474) (width 0.2) (layer "F.Cu") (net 25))
 (segment (start 149.249 72.78984) (end 149.56484 72.474) (width 0.2) (layer "F.Cu") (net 25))
 (segment (start 161.324 72.474) (end 162.35 73.5) (width 0.2) (layer "F.Cu") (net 25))
 (segment (start 149.8625 78.55) (end 149.249 77.9365) (width 0.2) (layer "F.Cu") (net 25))
 (segment (start 152.43516 72.474) (end 153.101 73.13984) (width 0.2) (layer "F.Cu") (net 25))
 (segment (start 128.249 86.943206) (end 128.776794 87.471) (width 0.2) (layer "F.Cu") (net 12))
 (segment (start 163.901 72.36484) (end 163.58516 72.049) (width 0.2) (layer "F.Cu") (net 12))
 (segment (start 163.58516 72.049) (end 136.256794 72.049) (width 0.2) (layer "F.Cu") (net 12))
 (segment (start 162 85) (end 162 76.53616) (width 0.2) (layer "F.Cu") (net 12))
 (segment (start 133.516 87.471) (end 134.25 86.737) (width 0.2) (layer "F.Cu") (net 12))
 (segment (start 162 76.53616) (end 163.901 74.63516) (width 0.2) (layer "F.Cu") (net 12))
 (segment (start 134.25 86.737) (end 134.25 85.8) (width 0.2) (layer "F.Cu") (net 12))
 (segment (start 163.0875 85.5) (end 162.5 85.5) (width 0.2) (layer "F.Cu") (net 12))
 (segment (start 162.5 85.5) (end 162 85) (width 0.2) (layer "F.Cu") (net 12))
 (segment (start 136.256794 72.049) (end 128.249 80.056794) (width 0.2) (layer "F.Cu") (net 12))
 (segment (start 128.776794 87.471) (end 133.516 87.471) (width 0.2) (layer "F.Cu") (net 12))
 (segment (start 128.249 80.056794) (end 128.249 86.943206) (width 0.2) (layer "F.Cu") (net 12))
 (segment (start 163.901 74.63516) (end 163.901 72.36484) (width 0.2) (layer "F.Cu") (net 12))
 (segment (start 132.75 82.137) (end 135.412 84.799) (width 0.2) (layer "F.Cu") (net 1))
 (segment (start 144.9515 84.799) (end 151.9225 91.77) (width 0.2) (layer "F.Cu") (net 1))
 (segment (start 135.412 84.799) (end 144.9515 84.799) (width 0.2) (layer "F.Cu") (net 1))
 (segment (start 132.75 81.2) (end 132.75 82.137) (width 0.2) (layer "F.Cu") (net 1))
 (segment (start 163.0875 92.5875) (end 167.5 97) (width 0.2) (layer "F.Cu") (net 26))
 (segment (start 167.5 97) (end 167.5 101) (width 0.2) (layer "F.Cu") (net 26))
 (segment (start 163.0875 92) (end 163.0875 92.5875) (width 0.2) (layer "F.Cu") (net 26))
 (segment (start 149.8625 80.45) (end 149.95 80.45) (width 0.2) (layer "F.Cu") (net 27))
 (segment (start 149.95 80.45) (end 150 80.5) (width 0.2) (layer "F.Cu") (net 27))
 (segment (start 146.5145 83.798) (end 146.5 83.798) (width 0.2) (layer "F.Cu") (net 27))
 (segment (start 149.8625 80.45) (end 146.5145 83.798) (width 0.2) (layer "F.Cu") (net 27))
 (via (at 146.5 83.798) (size 0.6) (drill 0.3) (layers "F.Cu" "B.Cu") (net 27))
 (segment (start 166.242 103.54) (end 167.5 103.54) (width 0.2) (layer "B.Cu") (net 27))
 (segment (start 146.5 83.798) (end 166.242 103.54) (width 0.2) (layer "B.Cu") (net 27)))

